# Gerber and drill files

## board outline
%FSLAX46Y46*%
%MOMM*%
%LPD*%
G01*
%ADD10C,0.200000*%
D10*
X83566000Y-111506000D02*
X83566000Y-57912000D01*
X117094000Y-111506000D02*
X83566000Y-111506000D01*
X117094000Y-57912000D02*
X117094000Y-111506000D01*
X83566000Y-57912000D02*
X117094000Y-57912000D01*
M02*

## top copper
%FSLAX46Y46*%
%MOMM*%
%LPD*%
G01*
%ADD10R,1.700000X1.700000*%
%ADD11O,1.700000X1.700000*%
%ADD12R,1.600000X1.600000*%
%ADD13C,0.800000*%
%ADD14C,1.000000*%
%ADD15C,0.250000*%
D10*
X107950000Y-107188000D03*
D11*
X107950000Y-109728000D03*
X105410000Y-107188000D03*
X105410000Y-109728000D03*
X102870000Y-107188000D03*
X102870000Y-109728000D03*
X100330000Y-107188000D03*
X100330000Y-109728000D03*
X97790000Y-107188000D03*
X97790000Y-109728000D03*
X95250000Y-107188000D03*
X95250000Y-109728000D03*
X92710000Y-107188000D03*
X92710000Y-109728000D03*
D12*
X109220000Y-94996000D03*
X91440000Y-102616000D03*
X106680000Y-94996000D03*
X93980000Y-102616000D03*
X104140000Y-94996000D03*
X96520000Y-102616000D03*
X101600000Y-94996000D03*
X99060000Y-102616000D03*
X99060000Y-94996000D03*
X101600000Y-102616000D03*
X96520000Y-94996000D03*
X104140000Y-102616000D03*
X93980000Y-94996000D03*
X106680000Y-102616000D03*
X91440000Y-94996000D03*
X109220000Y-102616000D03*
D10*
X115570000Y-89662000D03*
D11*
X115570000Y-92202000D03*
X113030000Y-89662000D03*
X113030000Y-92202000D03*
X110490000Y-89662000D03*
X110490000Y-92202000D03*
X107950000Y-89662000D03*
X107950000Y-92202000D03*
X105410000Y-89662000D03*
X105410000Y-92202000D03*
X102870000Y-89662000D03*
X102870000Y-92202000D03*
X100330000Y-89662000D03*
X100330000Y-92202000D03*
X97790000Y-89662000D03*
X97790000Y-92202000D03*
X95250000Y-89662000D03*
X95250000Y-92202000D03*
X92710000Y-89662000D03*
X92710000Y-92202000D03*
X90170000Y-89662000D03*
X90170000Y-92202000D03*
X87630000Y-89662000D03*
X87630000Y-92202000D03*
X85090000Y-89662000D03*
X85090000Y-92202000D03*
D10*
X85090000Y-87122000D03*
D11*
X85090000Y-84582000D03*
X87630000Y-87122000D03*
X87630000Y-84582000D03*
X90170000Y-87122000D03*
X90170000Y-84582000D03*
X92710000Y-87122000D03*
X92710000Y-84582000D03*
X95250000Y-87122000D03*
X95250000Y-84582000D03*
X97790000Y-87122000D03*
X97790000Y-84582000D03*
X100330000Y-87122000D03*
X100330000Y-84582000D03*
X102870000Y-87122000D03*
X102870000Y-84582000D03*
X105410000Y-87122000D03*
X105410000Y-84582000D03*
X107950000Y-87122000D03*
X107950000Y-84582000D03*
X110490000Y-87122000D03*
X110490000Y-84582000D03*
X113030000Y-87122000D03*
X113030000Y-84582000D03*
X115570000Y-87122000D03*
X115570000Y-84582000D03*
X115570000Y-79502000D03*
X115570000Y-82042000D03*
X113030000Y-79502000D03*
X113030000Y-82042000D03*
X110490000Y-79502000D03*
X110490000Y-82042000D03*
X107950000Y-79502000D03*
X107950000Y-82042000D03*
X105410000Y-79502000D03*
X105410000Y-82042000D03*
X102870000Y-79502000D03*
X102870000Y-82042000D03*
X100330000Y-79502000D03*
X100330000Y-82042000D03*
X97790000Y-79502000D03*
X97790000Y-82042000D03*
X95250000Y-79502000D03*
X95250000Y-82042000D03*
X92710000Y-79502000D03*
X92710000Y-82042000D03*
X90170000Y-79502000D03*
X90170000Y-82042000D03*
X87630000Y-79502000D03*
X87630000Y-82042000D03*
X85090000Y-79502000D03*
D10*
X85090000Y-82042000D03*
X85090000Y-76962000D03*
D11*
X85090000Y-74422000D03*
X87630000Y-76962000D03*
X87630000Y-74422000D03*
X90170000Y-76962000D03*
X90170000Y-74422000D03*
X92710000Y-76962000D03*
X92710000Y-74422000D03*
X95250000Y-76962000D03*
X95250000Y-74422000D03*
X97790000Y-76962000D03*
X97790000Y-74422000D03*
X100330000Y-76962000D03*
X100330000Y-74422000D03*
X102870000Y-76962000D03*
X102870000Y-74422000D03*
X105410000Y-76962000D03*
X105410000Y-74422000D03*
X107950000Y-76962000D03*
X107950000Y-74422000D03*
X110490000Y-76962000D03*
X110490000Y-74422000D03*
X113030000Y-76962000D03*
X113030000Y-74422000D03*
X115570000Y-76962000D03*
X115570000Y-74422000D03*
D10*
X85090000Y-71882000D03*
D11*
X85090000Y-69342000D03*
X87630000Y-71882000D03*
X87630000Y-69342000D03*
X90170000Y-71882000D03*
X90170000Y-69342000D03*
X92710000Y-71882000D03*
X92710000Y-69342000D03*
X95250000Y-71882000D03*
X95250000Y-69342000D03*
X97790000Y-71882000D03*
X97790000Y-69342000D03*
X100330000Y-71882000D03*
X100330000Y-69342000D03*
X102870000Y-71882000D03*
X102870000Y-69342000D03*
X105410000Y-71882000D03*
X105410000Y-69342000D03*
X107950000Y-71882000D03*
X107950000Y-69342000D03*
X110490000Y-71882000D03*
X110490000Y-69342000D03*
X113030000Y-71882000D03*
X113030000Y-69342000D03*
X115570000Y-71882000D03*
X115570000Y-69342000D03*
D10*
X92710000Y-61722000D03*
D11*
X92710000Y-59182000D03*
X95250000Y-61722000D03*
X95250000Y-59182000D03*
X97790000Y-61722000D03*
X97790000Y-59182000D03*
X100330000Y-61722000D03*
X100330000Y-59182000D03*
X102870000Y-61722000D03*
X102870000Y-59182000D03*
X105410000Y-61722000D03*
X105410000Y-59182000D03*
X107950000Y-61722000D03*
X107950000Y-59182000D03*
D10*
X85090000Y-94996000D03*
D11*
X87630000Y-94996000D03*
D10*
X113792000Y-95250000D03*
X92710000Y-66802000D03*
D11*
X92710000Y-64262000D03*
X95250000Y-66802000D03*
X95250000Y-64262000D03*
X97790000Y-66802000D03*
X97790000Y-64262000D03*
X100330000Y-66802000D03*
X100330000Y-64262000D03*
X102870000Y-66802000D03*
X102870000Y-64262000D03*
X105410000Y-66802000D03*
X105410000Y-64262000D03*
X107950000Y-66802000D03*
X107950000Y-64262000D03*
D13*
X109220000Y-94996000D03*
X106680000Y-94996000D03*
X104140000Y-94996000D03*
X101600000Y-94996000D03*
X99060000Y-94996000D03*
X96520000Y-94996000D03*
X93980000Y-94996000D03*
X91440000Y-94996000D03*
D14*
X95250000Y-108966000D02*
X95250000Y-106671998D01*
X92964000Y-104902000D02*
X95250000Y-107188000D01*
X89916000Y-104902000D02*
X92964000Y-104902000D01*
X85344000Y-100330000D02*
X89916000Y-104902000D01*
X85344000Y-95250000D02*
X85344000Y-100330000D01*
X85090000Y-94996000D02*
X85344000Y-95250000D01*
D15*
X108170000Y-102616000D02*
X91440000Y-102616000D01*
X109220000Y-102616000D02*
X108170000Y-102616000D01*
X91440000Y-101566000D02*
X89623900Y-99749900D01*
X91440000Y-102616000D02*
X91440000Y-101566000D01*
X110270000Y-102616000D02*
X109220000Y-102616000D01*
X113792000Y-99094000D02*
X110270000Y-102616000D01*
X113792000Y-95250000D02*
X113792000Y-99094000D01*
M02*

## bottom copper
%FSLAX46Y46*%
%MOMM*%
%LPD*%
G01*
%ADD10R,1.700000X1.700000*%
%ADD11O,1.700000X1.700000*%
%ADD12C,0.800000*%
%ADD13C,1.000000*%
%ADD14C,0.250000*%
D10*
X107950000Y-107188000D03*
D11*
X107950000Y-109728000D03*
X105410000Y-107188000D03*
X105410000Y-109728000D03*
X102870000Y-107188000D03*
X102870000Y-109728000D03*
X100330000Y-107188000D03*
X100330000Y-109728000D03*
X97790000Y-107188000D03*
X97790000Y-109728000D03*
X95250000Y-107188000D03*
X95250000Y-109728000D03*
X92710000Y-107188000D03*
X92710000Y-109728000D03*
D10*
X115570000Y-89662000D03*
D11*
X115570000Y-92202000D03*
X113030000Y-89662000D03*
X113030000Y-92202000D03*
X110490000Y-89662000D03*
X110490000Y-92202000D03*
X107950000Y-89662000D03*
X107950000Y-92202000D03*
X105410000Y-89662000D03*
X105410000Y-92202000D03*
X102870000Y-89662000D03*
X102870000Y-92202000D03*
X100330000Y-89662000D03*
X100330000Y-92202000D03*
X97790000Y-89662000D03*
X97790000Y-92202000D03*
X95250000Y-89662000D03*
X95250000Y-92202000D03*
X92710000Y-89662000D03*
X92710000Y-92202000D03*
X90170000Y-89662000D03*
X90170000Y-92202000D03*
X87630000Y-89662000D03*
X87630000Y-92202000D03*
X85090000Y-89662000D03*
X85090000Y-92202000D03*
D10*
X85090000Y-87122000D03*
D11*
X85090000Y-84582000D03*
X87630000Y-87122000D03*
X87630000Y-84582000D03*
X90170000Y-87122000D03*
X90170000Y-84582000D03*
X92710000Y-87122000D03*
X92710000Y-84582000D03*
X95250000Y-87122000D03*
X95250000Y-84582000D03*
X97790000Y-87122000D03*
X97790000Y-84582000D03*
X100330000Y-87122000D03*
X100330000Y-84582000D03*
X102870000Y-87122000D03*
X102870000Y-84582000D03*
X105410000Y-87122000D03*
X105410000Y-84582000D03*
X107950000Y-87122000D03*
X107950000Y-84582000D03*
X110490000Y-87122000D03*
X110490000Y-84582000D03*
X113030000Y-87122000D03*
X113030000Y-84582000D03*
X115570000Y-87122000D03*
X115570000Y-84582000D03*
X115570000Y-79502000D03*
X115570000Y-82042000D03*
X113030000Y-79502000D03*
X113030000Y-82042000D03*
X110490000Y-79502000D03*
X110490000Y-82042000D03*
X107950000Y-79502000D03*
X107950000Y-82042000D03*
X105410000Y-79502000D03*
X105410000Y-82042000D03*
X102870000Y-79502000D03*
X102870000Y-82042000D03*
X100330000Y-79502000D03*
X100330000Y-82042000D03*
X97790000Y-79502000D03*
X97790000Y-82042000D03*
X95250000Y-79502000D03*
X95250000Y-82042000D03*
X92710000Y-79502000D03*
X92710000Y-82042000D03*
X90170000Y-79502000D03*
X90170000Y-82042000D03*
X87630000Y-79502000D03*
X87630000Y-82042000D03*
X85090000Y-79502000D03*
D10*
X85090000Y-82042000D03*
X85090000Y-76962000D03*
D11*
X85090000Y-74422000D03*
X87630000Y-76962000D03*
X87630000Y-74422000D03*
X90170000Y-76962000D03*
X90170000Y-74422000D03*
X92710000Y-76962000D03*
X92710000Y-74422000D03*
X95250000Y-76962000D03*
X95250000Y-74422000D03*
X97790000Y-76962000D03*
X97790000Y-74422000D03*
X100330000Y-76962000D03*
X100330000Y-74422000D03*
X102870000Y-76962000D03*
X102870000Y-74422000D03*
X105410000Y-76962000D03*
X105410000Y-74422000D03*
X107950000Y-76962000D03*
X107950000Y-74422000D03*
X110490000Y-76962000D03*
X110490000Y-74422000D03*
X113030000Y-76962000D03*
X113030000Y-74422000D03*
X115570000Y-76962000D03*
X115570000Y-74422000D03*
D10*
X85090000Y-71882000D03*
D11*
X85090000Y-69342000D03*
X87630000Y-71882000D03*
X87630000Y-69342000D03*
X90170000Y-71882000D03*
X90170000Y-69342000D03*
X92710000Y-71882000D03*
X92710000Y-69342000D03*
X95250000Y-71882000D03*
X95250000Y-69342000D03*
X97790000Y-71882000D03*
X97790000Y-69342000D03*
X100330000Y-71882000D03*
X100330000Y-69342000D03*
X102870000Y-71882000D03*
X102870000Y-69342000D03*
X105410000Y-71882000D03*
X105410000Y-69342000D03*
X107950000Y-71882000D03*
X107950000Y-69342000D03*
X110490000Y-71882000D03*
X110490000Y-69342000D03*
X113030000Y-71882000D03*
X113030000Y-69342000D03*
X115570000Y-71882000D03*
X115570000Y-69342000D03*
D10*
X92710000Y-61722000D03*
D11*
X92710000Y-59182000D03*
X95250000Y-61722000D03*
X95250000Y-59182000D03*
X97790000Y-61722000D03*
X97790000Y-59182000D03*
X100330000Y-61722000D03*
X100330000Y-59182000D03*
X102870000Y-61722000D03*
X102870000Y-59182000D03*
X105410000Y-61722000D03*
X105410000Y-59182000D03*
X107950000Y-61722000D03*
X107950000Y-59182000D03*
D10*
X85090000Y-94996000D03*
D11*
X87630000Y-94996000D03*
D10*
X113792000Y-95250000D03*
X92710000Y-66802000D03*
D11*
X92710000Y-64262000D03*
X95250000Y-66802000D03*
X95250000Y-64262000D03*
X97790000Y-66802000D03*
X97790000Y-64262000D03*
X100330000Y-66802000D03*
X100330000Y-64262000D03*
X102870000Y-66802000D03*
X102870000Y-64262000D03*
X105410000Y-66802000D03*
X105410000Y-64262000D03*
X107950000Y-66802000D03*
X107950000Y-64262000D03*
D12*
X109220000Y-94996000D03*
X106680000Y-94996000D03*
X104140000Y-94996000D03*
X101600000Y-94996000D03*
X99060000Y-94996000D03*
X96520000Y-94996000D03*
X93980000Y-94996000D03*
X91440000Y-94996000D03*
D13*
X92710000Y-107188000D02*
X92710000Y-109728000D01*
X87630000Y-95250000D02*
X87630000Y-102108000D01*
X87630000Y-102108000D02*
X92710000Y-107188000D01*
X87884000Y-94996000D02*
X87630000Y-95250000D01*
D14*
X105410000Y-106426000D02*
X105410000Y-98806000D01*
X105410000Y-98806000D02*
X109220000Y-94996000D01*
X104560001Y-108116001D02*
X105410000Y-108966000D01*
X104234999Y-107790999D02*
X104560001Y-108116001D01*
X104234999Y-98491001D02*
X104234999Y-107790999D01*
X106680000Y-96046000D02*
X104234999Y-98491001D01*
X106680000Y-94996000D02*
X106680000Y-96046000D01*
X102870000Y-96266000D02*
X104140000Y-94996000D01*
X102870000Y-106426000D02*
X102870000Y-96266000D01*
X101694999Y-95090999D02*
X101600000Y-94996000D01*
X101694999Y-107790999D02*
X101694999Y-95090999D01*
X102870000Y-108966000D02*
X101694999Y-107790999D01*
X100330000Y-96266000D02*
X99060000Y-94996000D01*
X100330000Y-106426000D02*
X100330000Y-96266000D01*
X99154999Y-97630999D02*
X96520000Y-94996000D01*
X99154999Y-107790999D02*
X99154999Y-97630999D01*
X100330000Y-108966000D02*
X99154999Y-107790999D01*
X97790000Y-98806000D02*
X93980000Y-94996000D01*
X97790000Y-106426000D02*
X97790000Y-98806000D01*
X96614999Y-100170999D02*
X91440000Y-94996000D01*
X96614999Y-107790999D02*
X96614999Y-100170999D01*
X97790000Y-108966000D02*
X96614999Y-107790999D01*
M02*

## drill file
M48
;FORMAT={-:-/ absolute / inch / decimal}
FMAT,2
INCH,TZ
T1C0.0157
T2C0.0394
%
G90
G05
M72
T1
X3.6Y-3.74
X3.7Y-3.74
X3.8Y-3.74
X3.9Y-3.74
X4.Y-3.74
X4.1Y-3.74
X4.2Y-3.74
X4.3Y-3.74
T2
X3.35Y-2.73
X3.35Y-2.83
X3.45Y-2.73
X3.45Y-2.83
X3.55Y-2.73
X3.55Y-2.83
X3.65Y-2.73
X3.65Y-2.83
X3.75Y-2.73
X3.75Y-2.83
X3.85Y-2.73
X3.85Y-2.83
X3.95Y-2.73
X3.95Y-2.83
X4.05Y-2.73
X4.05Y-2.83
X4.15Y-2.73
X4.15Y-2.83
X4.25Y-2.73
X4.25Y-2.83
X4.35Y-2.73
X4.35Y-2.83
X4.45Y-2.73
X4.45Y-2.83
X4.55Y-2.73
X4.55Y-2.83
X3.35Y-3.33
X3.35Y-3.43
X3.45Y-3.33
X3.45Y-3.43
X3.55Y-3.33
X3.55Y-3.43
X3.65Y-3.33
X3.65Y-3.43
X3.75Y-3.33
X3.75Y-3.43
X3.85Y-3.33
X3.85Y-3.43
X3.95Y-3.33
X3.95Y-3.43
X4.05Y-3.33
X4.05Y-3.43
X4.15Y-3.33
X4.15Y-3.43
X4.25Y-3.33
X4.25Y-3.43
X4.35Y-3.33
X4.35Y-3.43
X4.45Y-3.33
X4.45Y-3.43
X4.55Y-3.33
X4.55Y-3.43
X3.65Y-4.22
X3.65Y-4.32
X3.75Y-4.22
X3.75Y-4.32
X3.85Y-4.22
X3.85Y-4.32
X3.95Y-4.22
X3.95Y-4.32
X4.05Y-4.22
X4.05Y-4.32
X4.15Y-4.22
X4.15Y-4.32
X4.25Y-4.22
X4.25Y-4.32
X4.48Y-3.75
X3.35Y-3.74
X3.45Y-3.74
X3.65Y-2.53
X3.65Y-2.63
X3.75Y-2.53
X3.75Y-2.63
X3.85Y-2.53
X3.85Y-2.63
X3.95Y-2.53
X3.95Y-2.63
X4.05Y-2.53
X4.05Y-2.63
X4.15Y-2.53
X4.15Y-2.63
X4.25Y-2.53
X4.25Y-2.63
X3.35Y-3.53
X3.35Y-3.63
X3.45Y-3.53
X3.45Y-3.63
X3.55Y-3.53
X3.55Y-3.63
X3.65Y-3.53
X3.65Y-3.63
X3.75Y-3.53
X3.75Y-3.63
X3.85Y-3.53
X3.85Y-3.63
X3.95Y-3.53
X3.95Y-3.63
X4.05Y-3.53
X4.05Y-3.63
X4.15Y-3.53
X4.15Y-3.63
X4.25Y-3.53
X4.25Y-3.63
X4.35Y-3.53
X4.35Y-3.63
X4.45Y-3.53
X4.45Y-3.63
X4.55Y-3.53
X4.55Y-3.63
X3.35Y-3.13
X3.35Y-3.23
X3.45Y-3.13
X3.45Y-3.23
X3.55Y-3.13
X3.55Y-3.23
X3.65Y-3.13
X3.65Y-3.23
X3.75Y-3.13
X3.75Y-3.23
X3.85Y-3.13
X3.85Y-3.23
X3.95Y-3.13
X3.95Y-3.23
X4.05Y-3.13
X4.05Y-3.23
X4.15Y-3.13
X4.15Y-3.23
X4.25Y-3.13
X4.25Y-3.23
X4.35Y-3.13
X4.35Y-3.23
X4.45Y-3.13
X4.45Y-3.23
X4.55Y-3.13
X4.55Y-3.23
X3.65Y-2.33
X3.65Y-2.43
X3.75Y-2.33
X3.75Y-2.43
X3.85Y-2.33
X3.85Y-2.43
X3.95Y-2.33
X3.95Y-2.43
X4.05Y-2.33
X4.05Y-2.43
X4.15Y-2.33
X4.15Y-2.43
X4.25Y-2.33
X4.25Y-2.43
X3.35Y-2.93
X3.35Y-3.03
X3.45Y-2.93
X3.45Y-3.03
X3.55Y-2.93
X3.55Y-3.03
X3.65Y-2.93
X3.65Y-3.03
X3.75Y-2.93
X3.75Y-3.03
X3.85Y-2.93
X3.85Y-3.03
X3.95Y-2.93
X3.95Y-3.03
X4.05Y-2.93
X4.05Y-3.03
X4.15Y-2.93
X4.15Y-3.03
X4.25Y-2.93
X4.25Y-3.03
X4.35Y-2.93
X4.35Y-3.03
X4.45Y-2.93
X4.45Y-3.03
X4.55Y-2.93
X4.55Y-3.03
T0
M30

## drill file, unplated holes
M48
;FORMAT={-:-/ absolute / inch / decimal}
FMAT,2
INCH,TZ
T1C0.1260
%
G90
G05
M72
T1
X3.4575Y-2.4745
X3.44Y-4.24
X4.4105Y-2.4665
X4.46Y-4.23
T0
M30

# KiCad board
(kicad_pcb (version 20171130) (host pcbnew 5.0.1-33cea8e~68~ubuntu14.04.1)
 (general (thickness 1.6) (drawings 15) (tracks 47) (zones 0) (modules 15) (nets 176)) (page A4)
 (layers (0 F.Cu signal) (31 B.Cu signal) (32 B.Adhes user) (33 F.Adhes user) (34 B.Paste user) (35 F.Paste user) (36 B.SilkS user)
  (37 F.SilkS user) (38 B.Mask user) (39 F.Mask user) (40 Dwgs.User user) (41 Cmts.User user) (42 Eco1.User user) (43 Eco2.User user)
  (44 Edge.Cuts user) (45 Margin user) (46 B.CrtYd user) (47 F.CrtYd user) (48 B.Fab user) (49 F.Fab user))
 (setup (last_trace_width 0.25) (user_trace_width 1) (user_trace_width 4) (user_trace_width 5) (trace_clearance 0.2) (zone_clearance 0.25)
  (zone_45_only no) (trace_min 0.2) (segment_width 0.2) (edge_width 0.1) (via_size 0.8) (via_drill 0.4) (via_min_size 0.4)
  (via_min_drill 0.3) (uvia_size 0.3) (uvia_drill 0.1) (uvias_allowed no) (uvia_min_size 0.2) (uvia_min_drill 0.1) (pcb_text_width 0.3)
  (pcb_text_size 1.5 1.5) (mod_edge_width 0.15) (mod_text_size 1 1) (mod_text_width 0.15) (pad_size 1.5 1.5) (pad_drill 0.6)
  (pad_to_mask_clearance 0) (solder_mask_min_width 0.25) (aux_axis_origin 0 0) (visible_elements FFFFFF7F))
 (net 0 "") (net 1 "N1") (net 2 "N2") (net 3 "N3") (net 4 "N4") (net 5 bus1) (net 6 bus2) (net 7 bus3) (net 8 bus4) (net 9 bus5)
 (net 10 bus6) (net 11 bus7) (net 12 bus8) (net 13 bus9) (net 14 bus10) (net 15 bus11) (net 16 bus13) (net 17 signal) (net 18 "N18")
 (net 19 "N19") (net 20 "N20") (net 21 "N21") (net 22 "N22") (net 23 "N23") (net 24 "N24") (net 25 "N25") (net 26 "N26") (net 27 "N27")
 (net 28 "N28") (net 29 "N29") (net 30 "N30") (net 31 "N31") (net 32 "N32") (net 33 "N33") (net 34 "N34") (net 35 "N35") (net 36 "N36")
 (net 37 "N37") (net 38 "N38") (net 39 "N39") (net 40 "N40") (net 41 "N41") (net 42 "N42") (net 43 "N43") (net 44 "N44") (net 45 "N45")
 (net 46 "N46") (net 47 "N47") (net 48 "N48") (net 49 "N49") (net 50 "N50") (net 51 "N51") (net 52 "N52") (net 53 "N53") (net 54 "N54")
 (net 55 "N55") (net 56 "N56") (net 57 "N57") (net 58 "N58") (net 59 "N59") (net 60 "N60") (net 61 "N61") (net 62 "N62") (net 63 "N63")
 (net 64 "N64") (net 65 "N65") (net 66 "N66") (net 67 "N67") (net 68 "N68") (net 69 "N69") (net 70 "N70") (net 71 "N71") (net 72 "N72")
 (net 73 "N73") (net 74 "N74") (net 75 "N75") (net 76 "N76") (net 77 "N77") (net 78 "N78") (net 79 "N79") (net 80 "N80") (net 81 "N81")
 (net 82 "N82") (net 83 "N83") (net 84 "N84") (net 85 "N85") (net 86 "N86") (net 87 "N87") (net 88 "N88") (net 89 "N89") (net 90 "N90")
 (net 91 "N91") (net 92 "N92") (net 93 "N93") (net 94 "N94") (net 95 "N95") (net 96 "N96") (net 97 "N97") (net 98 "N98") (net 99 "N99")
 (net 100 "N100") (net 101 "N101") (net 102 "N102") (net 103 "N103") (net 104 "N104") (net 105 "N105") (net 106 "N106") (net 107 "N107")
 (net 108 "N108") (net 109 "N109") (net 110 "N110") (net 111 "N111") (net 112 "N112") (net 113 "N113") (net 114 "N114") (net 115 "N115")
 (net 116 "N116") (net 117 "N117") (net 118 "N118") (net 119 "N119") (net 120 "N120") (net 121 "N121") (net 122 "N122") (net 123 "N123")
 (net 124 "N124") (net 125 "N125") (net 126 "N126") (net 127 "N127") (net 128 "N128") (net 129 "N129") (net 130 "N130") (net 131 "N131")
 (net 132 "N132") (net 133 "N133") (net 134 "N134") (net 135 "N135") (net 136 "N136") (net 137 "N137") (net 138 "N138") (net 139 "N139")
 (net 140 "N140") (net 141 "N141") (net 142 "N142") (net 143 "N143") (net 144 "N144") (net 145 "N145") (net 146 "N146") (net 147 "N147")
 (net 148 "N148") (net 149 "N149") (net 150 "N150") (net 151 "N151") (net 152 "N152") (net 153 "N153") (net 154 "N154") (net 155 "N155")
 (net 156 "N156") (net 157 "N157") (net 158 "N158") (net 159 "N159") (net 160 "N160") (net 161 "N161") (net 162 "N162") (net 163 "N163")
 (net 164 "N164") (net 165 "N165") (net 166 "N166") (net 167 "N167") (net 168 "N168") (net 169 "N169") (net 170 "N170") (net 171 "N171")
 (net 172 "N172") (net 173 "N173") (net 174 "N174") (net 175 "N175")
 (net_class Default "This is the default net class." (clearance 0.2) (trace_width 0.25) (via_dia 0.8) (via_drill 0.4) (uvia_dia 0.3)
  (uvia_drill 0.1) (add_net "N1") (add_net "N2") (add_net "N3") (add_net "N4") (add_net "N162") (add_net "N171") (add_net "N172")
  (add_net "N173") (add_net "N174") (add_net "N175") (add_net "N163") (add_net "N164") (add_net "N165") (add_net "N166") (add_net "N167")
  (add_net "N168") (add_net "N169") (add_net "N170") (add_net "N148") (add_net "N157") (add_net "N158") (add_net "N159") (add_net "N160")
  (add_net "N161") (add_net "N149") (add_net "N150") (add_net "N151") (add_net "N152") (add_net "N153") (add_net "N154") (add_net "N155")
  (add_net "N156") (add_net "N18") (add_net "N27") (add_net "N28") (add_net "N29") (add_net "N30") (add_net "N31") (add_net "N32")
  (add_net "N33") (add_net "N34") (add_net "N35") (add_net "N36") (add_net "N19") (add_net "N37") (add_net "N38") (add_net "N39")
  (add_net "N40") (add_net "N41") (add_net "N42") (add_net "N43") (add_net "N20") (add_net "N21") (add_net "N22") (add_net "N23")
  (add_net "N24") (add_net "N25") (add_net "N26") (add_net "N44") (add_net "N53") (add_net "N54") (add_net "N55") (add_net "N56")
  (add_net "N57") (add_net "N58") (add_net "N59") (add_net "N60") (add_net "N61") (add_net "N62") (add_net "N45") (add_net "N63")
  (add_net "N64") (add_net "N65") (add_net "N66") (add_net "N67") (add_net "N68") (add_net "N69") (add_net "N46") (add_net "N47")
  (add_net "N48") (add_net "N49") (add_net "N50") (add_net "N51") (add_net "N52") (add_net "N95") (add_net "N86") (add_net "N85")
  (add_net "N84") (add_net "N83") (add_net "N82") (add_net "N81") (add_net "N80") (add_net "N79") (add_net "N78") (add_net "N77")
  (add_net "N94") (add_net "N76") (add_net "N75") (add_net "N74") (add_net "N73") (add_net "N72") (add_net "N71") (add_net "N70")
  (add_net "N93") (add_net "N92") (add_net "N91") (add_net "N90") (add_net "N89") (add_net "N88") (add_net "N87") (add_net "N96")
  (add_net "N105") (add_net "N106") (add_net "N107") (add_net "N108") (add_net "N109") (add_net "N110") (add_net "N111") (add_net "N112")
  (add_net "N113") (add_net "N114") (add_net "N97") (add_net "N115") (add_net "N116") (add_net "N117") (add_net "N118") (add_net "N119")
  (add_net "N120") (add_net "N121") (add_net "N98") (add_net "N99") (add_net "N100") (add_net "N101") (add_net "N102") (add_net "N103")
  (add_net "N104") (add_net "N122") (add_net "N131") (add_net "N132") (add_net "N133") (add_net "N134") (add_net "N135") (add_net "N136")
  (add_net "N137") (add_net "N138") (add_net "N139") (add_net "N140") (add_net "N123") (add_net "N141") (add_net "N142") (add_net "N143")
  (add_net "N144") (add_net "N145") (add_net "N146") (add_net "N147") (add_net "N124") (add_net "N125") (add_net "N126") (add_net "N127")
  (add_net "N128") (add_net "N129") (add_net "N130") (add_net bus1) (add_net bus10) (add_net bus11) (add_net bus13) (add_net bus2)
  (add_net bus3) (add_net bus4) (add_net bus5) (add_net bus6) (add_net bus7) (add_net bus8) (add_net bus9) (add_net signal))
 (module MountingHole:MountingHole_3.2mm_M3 (layer F.Cu) (at 87.376 107.696)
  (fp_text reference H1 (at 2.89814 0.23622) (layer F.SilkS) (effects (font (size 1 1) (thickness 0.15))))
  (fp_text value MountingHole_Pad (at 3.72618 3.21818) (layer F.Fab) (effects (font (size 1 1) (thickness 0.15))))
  (pad 1 np_thru_hole circle (at 0 0) (size 3.2 3.2) (drill 3.2) (layers *.Cu *.Mask) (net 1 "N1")))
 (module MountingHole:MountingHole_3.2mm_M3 (layer F.Cu) (at 113.284 107.442)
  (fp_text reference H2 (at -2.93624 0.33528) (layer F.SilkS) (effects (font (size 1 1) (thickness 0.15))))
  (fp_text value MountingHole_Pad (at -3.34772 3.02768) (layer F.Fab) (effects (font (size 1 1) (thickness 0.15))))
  (pad 1 np_thru_hole circle (at 0 0) (size 3.2 3.2) (drill 3.2) (layers *.Cu *.Mask) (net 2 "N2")))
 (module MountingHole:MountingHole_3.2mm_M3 (layer F.Cu) (at 112.0267 62.6491)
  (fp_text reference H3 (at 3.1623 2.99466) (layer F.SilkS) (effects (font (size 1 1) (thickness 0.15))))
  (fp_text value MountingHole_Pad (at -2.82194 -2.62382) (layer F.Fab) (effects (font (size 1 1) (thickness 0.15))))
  (pad 1 np_thru_hole circle (at 0 0) (size 3.2 3.2) (drill 3.2) (layers *.Cu *.Mask) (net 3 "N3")))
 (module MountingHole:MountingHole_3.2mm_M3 (layer F.Cu) (at 87.8205 62.8523)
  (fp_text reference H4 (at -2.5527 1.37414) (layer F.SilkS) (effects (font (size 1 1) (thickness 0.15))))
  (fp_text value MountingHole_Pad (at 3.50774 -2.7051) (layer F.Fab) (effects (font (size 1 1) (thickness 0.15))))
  (pad 1 np_thru_hole circle (at 0 0) (size 3.2 3.2) (drill 3.2) (layers *.Cu *.Mask) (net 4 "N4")))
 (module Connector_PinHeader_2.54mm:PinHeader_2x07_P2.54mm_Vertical (layer F.Cu) (at 107.95 107.188 270)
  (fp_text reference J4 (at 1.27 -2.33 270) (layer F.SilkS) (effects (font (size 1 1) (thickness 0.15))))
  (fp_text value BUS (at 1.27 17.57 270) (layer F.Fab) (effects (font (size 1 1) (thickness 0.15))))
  (pad 1 thru_hole rect (at 0 0 270) (size 1.7 1.7) (drill 1) (layers *.Cu *.Mask) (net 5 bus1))
  (pad 2 thru_hole oval (at 2.54 0 270) (size 1.7 1.7) (drill 1) (layers *.Cu *.Mask) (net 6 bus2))
  (pad 3 thru_hole oval (at 0 2.54 270) (size 1.7 1.7) (drill 1) (layers *.Cu *.Mask) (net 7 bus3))
  (pad 4 thru_hole oval (at 2.54 2.54 270) (size 1.7 1.7) (drill 1) (layers *.Cu *.Mask) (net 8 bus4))
  (pad 5 thru_hole oval (at 0 5.08 270) (size 1.7 1.7) (drill 1) (layers *.Cu *.Mask) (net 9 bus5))
  (pad 6 thru_hole oval (at 2.54 5.08 270) (size 1.7 1.7) (drill 1) (layers *.Cu *.Mask) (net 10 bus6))
  (pad 7 thru_hole oval (at 0 7.62 270) (size 1.7 1.7) (drill 1) (layers *.Cu *.Mask) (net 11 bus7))
  (pad 8 thru_hole oval (at 2.54 7.62 270) (size 1.7 1.7) (drill 1) (layers *.Cu *.Mask) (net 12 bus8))
  (pad 9 thru_hole oval (at 0 10.16 270) (size 1.7 1.7) (drill 1) (layers *.Cu *.Mask) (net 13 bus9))
  (pad 10 thru_hole oval (at 2.54 10.16 270) (size 1.7 1.7) (drill 1) (layers *.Cu *.Mask) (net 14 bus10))
  (pad 11 thru_hole oval (at 0 12.7 270) (size 1.7 1.7) (drill 1) (layers *.Cu *.Mask) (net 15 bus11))
  (pad 12 thru_hole oval (at 2.54 12.7 270) (size 1.7 1.7) (drill 1) (layers *.Cu *.Mask) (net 15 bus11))
  (pad 13 thru_hole oval (at 0 15.24 270) (size 1.7 1.7) (drill 1) (layers *.Cu *.Mask) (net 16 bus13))
  (pad 14 thru_hole oval (at 2.54 15.24 270) (size 1.7 1.7) (drill 1) (layers *.Cu *.Mask) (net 16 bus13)))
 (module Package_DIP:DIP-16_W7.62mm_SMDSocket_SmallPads (layer F.Cu) (at 100.33 98.806 270)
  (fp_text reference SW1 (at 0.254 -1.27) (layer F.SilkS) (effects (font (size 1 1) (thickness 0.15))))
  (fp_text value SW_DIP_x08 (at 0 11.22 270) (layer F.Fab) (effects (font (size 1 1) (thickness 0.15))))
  (pad 1 smd rect (at -3.81 -8.89 270) (size 1.6 1.6) (layers F.Cu F.Paste F.Mask) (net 7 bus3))
  (pad 9 smd rect (at 3.81 8.89 270) (size 1.6 1.6) (layers F.Cu F.Paste F.Mask) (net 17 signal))
  (pad 2 smd rect (at -3.81 -6.35 270) (size 1.6 1.6) (layers F.Cu F.Paste F.Mask) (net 8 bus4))
  (pad 10 smd rect (at 3.81 6.35 270) (size 1.6 1.6) (layers F.Cu F.Paste F.Mask) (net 17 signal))
  (pad 3 smd rect (at -3.81 -3.81 270) (size 1.6 1.6) (layers F.Cu F.Paste F.Mask) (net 9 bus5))
  (pad 11 smd rect (at 3.81 3.81 270) (size 1.6 1.6) (layers F.Cu F.Paste F.Mask) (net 17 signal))
  (pad 4 smd rect (at -3.81 -1.27 270) (size 1.6 1.6) (layers F.Cu F.Paste F.Mask) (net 10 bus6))
  (pad 12 smd rect (at 3.81 1.27 270) (size 1.6 1.6) (layers F.Cu F.Paste F.Mask) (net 17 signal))
  (pad 5 smd rect (at -3.81 1.27 270) (size 1.6 1.6) (layers F.Cu F.Paste F.Mask) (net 11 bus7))
  (pad 13 smd rect (at 3.81 -1.27 270) (size 1.6 1.6) (layers F.Cu F.Paste F.Mask) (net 17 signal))
  (pad 6 smd rect (at -3.81 3.81 270) (size 1.6 1.6) (layers F.Cu F.Paste F.Mask) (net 12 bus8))
  (pad 14 smd rect (at 3.81 -3.81 270) (size 1.6 1.6) (layers F.Cu F.Paste F.Mask) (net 17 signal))
  (pad 7 smd rect (at -3.81 6.35 270) (size 1.6 1.6) (layers F.Cu F.Paste F.Mask) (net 13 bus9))
  (pad 15 smd rect (at 3.81 -6.35 270) (size 1.6 1.6) (layers F.Cu F.Paste F.Mask) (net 17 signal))
  (pad 8 smd rect (at -3.81 8.89 270) (size 1.6 1.6) (layers F.Cu F.Paste F.Mask) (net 14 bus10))
  (pad 16 smd rect (at 3.81 -8.89 270) (size 1.6 1.6) (layers F.Cu F.Paste F.Mask) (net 17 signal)))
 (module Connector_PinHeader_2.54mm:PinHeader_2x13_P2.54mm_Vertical (layer F.Cu) (at 115.57 89.662 270)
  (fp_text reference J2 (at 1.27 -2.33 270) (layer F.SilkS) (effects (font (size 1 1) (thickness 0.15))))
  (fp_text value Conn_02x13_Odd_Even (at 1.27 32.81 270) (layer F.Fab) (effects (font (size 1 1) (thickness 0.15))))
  (pad 1 thru_hole rect (at 0 0 270) (size 1.7 1.7) (drill 1) (layers *.Cu *.Mask) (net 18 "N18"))
  (pad 2 thru_hole oval (at 2.54 0 270) (size 1.7 1.7) (drill 1) (layers *.Cu *.Mask) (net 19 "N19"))
  (pad 3 thru_hole oval (at 0 2.54 270) (size 1.7 1.7) (drill 1) (layers *.Cu *.Mask) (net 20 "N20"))
  (pad 4 thru_hole oval (at 2.54 2.54 270) (size 1.7 1.7) (drill 1) (layers *.Cu *.Mask) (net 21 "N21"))
  (pad 5 thru_hole oval (at 0 5.08 270) (size 1.7 1.7) (drill 1) (layers *.Cu *.Mask) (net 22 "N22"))
  (pad 6 thru_hole oval (at 2.54 5.08 270) (size 1.7 1.7) (drill 1) (layers *.Cu *.Mask) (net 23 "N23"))
  (pad 7 thru_hole oval (at 0 7.62 270) (size 1.7 1.7) (drill 1) (layers *.Cu *.Mask) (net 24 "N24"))
  (pad 8 thru_hole oval (at 2.54 7.62 270) (size 1.7 1.7) (drill 1) (layers *.Cu *.Mask) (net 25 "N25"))
  (pad 9 thru_hole oval (at 0 10.16 270) (size 1.7 1.7) (drill 1) (layers *.Cu *.Mask) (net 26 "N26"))
  (pad 10 thru_hole oval (at 2.54 10.16 270) (size 1.7 1.7) (drill 1) (layers *.Cu *.Mask) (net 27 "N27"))
  (pad 11 thru_hole oval (at 0 12.7 270) (size 1.7 1.7) (drill 1) (layers *.Cu *.Mask) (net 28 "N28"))
  (pad 12 thru_hole oval (at 2.54 12.7 270) (size 1.7 1.7) (drill 1) (layers *.Cu *.Mask) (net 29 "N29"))
  (pad 13 thru_hole oval (at 0 15.24 270) (size 1.7 1.7) (drill 1) (layers *.Cu *.Mask) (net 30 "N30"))
  (pad 14 thru_hole oval (at 2.54 15.24 270) (size 1.7 1.7) (drill 1) (layers *.Cu *.Mask) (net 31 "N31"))
  (pad 15 thru_hole oval (at 0 17.78 270) (size 1.7 1.7) (drill 1) (layers *.Cu *.Mask) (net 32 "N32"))
  (pad 16 thru_hole oval (at 2.54 17.78 270) (size 1.7 1.7) (drill 1) (layers *.Cu *.Mask) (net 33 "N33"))
  (pad 17 thru_hole oval (at 0 20.32 270) (size 1.7 1.7) (drill 1) (layers *.Cu *.Mask) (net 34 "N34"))
  (pad 18 thru_hole oval (at 2.54 20.32 270) (size 1.7 1.7) (drill 1) (layers *.Cu *.Mask) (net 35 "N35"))
  (pad 19 thru_hole oval (at 0 22.86 270) (size 1.7 1.7) (drill 1) (layers *.Cu *.Mask) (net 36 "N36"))
  (pad 20 thru_hole oval (at 2.54 22.86 270) (size 1.7 1.7) (drill 1) (layers *.Cu *.Mask) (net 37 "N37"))
  (pad 21 thru_hole oval (at 0 25.4 270) (size 1.7 1.7) (drill 1) (layers *.Cu *.Mask) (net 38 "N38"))
  (pad 22 thru_hole oval (at 2.54 25.4 270) (size 1.7 1.7) (drill 1) (layers *.Cu *.Mask) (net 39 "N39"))
  (pad 23 thru_hole oval (at 0 27.94 270) (size 1.7 1.7) (drill 1) (layers *.Cu *.Mask) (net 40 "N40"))
  (pad 24 thru_hole oval (at 2.54 27.94 270) (size 1.7 1.7) (drill 1) (layers *.Cu *.Mask) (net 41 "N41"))
  (pad 25 thru_hole oval (at 0 30.48 270) (size 1.7 1.7) (drill 1) (layers *.Cu *.Mask) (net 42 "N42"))
  (pad 26 thru_hole oval (at 2.54 30.48 270) (size 1.7 1.7) (drill 1) (layers *.Cu *.Mask) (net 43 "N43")))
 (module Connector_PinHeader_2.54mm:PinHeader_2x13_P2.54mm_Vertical (layer F.Cu) (at 85.09 87.122 90)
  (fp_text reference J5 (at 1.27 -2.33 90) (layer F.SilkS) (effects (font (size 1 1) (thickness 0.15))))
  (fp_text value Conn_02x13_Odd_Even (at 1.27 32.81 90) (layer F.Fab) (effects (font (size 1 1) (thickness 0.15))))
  (pad 1 thru_hole rect (at 0 0 90) (size 1.7 1.7) (drill 1) (layers *.Cu *.Mask) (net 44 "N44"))
  (pad 2 thru_hole oval (at 2.54 0 90) (size 1.7 1.7) (drill 1) (layers *.Cu *.Mask) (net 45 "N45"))
  (pad 3 thru_hole oval (at 0 2.54 90) (size 1.7 1.7) (drill 1) (layers *.Cu *.Mask) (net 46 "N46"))
  (pad 4 thru_hole oval (at 2.54 2.54 90) (size 1.7 1.7) (drill 1) (layers *.Cu *.Mask) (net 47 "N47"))
  (pad 5 thru_hole oval (at 0 5.08 90) (size 1.7 1.7) (drill 1) (layers *.Cu *.Mask) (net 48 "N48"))
  (pad 6 thru_hole oval (at 2.54 5.08 90) (size 1.7 1.7) (drill 1) (layers *.Cu *.Mask) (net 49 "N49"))
  (pad 7 thru_hole oval (at 0 7.62 90) (size 1.7 1.7) (drill 1) (layers *.Cu *.Mask) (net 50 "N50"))
  (pad 8 thru_hole oval (at 2.54 7.62 90) (size 1.7 1.7) (drill 1) (layers *.Cu *.Mask) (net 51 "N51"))
  (pad 9 thru_hole oval (at 0 10.16 90) (size 1.7 1.7) (drill 1) (layers *.Cu *.Mask) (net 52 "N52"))
  (pad 10 thru_hole oval (at 2.54 10.16 90) (size 1.7 1.7) (drill 1) (layers *.Cu *.Mask) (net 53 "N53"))
  (pad 11 thru_hole oval (at 0 12.7 90) (size 1.7 1.7) (drill 1) (layers *.Cu *.Mask) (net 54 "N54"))
  (pad 12 thru_hole oval (at 2.54 12.7 90) (size 1.7 1.7) (drill 1) (layers *.Cu *.Mask) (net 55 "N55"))
  (pad 13 thru_hole oval (at 0 15.24 90) (size 1.7 1.7) (drill 1) (layers *.Cu *.Mask) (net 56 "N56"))
  (pad 14 thru_hole oval (at 2.54 15.24 90) (size 1.7 1.7) (drill 1) (layers *.Cu *.Mask) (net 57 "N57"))
  (pad 15 thru_hole oval (at 0 17.78 90) (size 1.7 1.7) (drill 1) (layers *.Cu *.Mask) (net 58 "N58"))
  (pad 16 thru_hole oval (at 2.54 17.78 90) (size 1.7 1.7) (drill 1) (layers *.Cu *.Mask) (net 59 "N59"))
  (pad 17 thru_hole oval (at 0 20.32 90) (size 1.7 1.7) (drill 1) (layers *.Cu *.Mask) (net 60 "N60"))
  (pad 18 thru_hole oval (at 2.54 20.32 90) (size 1.7 1.7) (drill 1) (layers *.Cu *.Mask) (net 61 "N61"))
  (pad 19 thru_hole oval (at 0 22.86 90) (size 1.7 1.7) (drill 1) (layers *.Cu *.Mask) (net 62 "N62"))
  (pad 20 thru_hole oval (at 2.54 22.86 90) (size 1.7 1.7) (drill 1) (layers *.Cu *.Mask) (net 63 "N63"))
  (pad 21 thru_hole oval (at 0 25.4 90) (size 1.7 1.7) (drill 1) (layers *.Cu *.Mask) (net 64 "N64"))
  (pad 22 thru_hole oval (at 2.54 25.4 90) (size 1.7 1.7) (drill 1) (layers *.Cu *.Mask) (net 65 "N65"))
  (pad 23 thru_hole oval (at 0 27.94 90) (size 1.7 1.7) (drill 1) (layers *.Cu *.Mask) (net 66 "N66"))
  (pad 24 thru_hole oval (at 2.54 27.94 90) (size 1.7 1.7) (drill 1) (layers *.Cu *.Mask) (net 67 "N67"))
  (pad 25 thru_hole oval (at 0 30.48 90) (size 1.7 1.7) (drill 1) (layers *.Cu *.Mask) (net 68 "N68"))
  (pad 26 thru_hole oval (at 2.54 30.48 90) (size 1.7 1.7) (drill 1) (layers *.Cu *.Mask) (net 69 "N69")))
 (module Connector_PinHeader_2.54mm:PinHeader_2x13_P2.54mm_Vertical (layer F.Cu) (at 85.09 82.042 90)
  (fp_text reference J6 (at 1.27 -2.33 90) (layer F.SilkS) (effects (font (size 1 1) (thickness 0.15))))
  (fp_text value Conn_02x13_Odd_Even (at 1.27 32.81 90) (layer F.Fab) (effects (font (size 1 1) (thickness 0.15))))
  (pad 26 thru_hole oval (at 2.54 30.48 90) (size 1.7 1.7) (drill 1) (layers *.Cu *.Mask) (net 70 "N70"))
  (pad 25 thru_hole oval (at 0 30.48 90) (size 1.7 1.7) (drill 1) (layers *.Cu *.Mask) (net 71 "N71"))
  (pad 24 thru_hole oval (at 2.54 27.94 90) (size 1.7 1.7) (drill 1) (layers *.Cu *.Mask) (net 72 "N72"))
  (pad 23 thru_hole oval (at 0 27.94 90) (size 1.7 1.7) (drill 1) (layers *.Cu *.Mask) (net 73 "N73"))
  (pad 22 thru_hole oval (at 2.54 25.4 90) (size 1.7 1.7) (drill 1) (layers *.Cu *.Mask) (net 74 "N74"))
  (pad 21 thru_hole oval (at 0 25.4 90) (size 1.7 1.7) (drill 1) (layers *.Cu *.Mask) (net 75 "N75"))
  (pad 20 thru_hole oval (at 2.54 22.86 90) (size 1.7 1.7) (drill 1) (layers *.Cu *.Mask) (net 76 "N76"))
  (pad 19 thru_hole oval (at 0 22.86 90) (size 1.7 1.7) (drill 1) (layers *.Cu *.Mask) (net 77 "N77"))
  (pad 18 thru_hole oval (at 2.54 20.32 90) (size 1.7 1.7) (drill 1) (layers *.Cu *.Mask) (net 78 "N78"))
  (pad 17 thru_hole oval (at 0 20.32 90) (size 1.7 1.7) (drill 1) (layers *.Cu *.Mask) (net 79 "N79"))
  (pad 16 thru_hole oval (at 2.54 17.78 90) (size 1.7 1.7) (drill 1) (layers *.Cu *.Mask) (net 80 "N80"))
  (pad 15 thru_hole oval (at 0 17.78 90) (size 1.7 1.7) (drill 1) (layers *.Cu *.Mask) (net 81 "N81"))
  (pad 14 thru_hole oval (at 2.54 15.24 90) (size 1.7 1.7) (drill 1) (layers *.Cu *.Mask) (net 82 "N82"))
  (pad 13 thru_hole oval (at 0 15.24 90) (size 1.7 1.7) (drill 1) (layers *.Cu *.Mask) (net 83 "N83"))
  (pad 12 thru_hole oval (at 2.54 12.7 90) (size 1.7 1.7) (drill 1) (layers *.Cu *.Mask) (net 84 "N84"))
  (pad 11 thru_hole oval (at 0 12.7 90) (size 1.7 1.7) (drill 1) (layers *.Cu *.Mask) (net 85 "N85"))
  (pad 10 thru_hole oval (at 2.54 10.16 90) (size 1.7 1.7) (drill 1) (layers *.Cu *.Mask) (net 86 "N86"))
  (pad 9 thru_hole oval (at 0 10.16 90) (size 1.7 1.7) (drill 1) (layers *.Cu *.Mask) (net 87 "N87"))
  (pad 8 thru_hole oval (at 2.54 7.62 90) (size 1.7 1.7) (drill 1) (layers *.Cu *.Mask) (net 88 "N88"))
  (pad 7 thru_hole oval (at 0 7.62 90) (size 1.7 1.7) (drill 1) (layers *.Cu *.Mask) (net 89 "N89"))
  (pad 6 thru_hole oval (at 2.54 5.08 90) (size 1.7 1.7) (drill 1) (layers *.Cu *.Mask) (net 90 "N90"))
  (pad 5 thru_hole oval (at 0 5.08 90) (size 1.7 1.7) (drill 1) (layers *.Cu *.Mask) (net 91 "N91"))
  (pad 4 thru_hole oval (at 2.54 2.54 90) (size 1.7 1.7) (drill 1) (layers *.Cu *.Mask) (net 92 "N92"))
  (pad 3 thru_hole oval (at 0 2.54 90) (size 1.7 1.7) (drill 1) (layers *.Cu *.Mask) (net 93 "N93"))
  (pad 2 thru_hole oval (at 2.54 0 90) (size 1.7 1.7) (drill 1) (layers *.Cu *.Mask) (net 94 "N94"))
  (pad 1 thru_hole rect (at 0 0 90) (size 1.7 1.7) (drill 1) (layers *.Cu *.Mask) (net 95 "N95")))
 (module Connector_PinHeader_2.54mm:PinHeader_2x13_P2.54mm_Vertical (layer F.Cu) (at 85.09 76.962 90)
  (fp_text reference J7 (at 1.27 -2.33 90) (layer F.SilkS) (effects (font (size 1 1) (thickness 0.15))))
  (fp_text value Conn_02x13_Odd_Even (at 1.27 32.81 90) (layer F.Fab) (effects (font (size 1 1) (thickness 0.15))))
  (pad 1 thru_hole rect (at 0 0 90) (size 1.7 1.7) (drill 1) (layers *.Cu *.Mask) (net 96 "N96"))
  (pad 2 thru_hole oval (at 2.54 0 90) (size 1.7 1.7) (drill 1) (layers *.Cu *.Mask) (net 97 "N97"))
  (pad 3 thru_hole oval (at 0 2.54 90) (size 1.7 1.7) (drill 1) (layers *.Cu *.Mask) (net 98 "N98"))
  (pad 4 thru_hole oval (at 2.54 2.54 90) (size 1.7 1.7) (drill 1) (layers *.Cu *.Mask) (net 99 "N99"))
  (pad 5 thru_hole oval (at 0 5.08 90) (size 1.7 1.7) (drill 1) (layers *.Cu *.Mask) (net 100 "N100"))
  (pad 6 thru_hole oval (at 2.54 5.08 90) (size 1.7 1.7) (drill 1) (layers *.Cu *.Mask) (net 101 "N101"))
  (pad 7 thru_hole oval (at 0 7.62 90) (size 1.7 1.7) (drill 1) (layers *.Cu *.Mask) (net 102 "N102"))
  (pad 8 thru_hole oval (at 2.54 7.62 90) (size 1.7 1.7) (drill 1) (layers *.Cu *.Mask) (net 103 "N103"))
  (pad 9 thru_hole oval (at 0 10.16 90) (size 1.7 1.7) (drill 1) (layers *.Cu *.Mask) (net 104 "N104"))
  (pad 10 thru_hole oval (at 2.54 10.16 90) (size 1.7 1.7) (drill 1) (layers *.Cu *.Mask) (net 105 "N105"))
  (pad 11 thru_hole oval (at 0 12.7 90) (size 1.7 1.7) (drill 1) (layers *.Cu *.Mask) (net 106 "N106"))
  (pad 12 thru_hole oval (at 2.54 12.7 90) (size 1.7 1.7) (drill 1) (layers *.Cu *.Mask) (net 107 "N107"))
  (pad 13 thru_hole oval (at 0 15.24 90) (size 1.7 1.7) (drill 1) (layers *.Cu *.Mask) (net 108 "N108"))
  (pad 14 thru_hole oval (at 2.54 15.24 90) (size 1.7 1.7) (drill 1) (layers *.Cu *.Mask) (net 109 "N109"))
  (pad 15 thru_hole oval (at 0 17.78 90) (size 1.7 1.7) (drill 1) (layers *.Cu *.Mask) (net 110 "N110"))
  (pad 16 thru_hole oval (at 2.54 17.78 90) (size 1.7 1.7) (drill 1) (layers *.Cu *.Mask) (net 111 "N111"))
  (pad 17 thru_hole oval (at 0 20.32 90) (size 1.7 1.7) (drill 1) (layers *.Cu *.Mask) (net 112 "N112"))
  (pad 18 thru_hole oval (at 2.54 20.32 90) (size 1.7 1.7) (drill 1) (layers *.Cu *.Mask) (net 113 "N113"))
  (pad 19 thru_hole oval (at 0 22.86 90) (size 1.7 1.7) (drill 1) (layers *.Cu *.Mask) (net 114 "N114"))
  (pad 20 thru_hole oval (at 2.54 22.86 90) (size 1.7 1.7) (drill 1) (layers *.Cu *.Mask) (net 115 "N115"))
  (pad 21 thru_hole oval (at 0 25.4 90) (size 1.7 1.7) (drill 1) (layers *.Cu *.Mask) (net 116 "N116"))
  (pad 22 thru_hole oval (at 2.54 25.4 90) (size 1.7 1.7) (drill 1) (layers *.Cu *.Mask) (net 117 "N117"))
  (pad 23 thru_hole oval (at 0 27.94 90) (size 1.7 1.7) (drill 1) (layers *.Cu *.Mask) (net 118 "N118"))
  (pad 24 thru_hole oval (at 2.54 27.94 90) (size 1.7 1.7) (drill 1) (layers *.Cu *.Mask) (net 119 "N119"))
  (pad 25 thru_hole oval (at 0 30.48 90) (size 1.7 1.7) (drill 1) (layers *.Cu *.Mask) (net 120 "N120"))
  (pad 26 thru_hole oval (at 2.54 30.48 90) (size 1.7 1.7) (drill 1) (layers *.Cu *.Mask) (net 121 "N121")))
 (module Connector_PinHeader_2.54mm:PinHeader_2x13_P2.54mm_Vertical (layer F.Cu) (at 85.09 71.882 90)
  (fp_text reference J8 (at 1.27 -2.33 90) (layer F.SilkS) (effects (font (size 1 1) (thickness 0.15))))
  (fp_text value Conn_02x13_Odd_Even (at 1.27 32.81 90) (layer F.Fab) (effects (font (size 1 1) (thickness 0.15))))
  (pad 1 thru_hole rect (at 0 0 90) (size 1.7 1.7) (drill 1) (layers *.Cu *.Mask) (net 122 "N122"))
  (pad 2 thru_hole oval (at 2.54 0 90) (size 1.7 1.7) (drill 1) (layers *.Cu *.Mask) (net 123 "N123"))
  (pad 3 thru_hole oval (at 0 2.54 90) (size 1.7 1.7) (drill 1) (layers *.Cu *.Mask) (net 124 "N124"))
  (pad 4 thru_hole oval (at 2.54 2.54 90) (size 1.7 1.7) (drill 1) (layers *.Cu *.Mask) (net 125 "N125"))
  (pad 5 thru_hole oval (at 0 5.08 90) (size 1.7 1.7) (drill 1) (layers *.Cu *.Mask) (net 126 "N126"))
  (pad 6 thru_hole oval (at 2.54 5.08 90) (size 1.7 1.7) (drill 1) (layers *.Cu *.Mask) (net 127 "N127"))
  (pad 7 thru_hole oval (at 0 7.62 90) (size 1.7 1.7) (drill 1) (layers *.Cu *.Mask) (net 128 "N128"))
  (pad 8 thru_hole oval (at 2.54 7.62 90) (size 1.7 1.7) (drill 1) (layers *.Cu *.Mask) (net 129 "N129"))
  (pad 9 thru_hole oval (at 0 10.16 90) (size 1.7 1.7) (drill 1) (layers *.Cu *.Mask) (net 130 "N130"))
  (pad 10 thru_hole oval (at 2.54 10.16 90) (size 1.7 1.7) (drill 1) (layers *.Cu *.Mask) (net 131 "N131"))
  (pad 11 thru_hole oval (at 0 12.7 90) (size 1.7 1.7) (drill 1) (layers *.Cu *.Mask) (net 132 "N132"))
  (pad 12 thru_hole oval (at 2.54 12.7 90) (size 1.7 1.7) (drill 1) (layers *.Cu *.Mask) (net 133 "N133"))
  (pad 13 thru_hole oval (at 0 15.24 90) (size 1.7 1.7) (drill 1) (layers *.Cu *.Mask) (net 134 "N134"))
  (pad 14 thru_hole oval (at 2.54 15.24 90) (size 1.7 1.7) (drill 1) (layers *.Cu *.Mask) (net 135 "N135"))
  (pad 15 thru_hole oval (at 0 17.78 90) (size 1.7 1.7) (drill 1) (layers *.Cu *.Mask) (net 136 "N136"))
  (pad 16 thru_hole oval (at 2.54 17.78 90) (size 1.7 1.7) (drill 1) (layers *.Cu *.Mask) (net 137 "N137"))
  (pad 17 thru_hole oval (at 0 20.32 90) (size 1.7 1.7) (drill 1) (layers *.Cu *.Mask) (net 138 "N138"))
  (pad 18 thru_hole oval (at 2.54 20.32 90) (size 1.7 1.7) (drill 1) (layers *.Cu *.Mask) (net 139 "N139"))
  (pad 19 thru_hole oval (at 0 22.86 90) (size 1.7 1.7) (drill 1) (layers *.Cu *.Mask) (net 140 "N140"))
  (pad 20 thru_hole oval (at 2.54 22.86 90) (size 1.7 1.7) (drill 1) (layers *.Cu *.Mask) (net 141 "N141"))
  (pad 21 thru_hole oval (at 0 25.4 90) (size 1.7 1.7) (drill 1) (layers *.Cu *.Mask) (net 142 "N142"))
  (pad 22 thru_hole oval (at 2.54 25.4 90) (size 1.7 1.7) (drill 1) (layers *.Cu *.Mask) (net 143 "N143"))
  (pad 23 thru_hole oval (at 0 27.94 90) (size 1.7 1.7) (drill 1) (layers *.Cu *.Mask) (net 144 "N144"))
  (pad 24 thru_hole oval (at 2.54 27.94 90) (size 1.7 1.7) (drill 1) (layers *.Cu *.Mask) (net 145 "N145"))
  (pad 25 thru_hole oval (at 0 30.48 90) (size 1.7 1.7) (drill 1) (layers *.Cu *.Mask) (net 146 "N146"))
  (pad 26 thru_hole oval (at 2.54 30.48 90) (size 1.7 1.7) (drill 1) (layers *.Cu *.Mask) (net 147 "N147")))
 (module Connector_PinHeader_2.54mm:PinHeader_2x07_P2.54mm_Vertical (layer F.Cu) (at 92.71 61.722 90)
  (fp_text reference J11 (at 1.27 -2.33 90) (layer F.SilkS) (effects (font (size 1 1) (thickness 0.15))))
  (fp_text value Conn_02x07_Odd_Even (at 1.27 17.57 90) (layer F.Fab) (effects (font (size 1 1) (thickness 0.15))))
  (pad 1 thru_hole rect (at 0 0 90) (size 1.7 1.7) (drill 1) (layers *.Cu *.Mask) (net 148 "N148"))
  (pad 2 thru_hole oval (at 2.54 0 90) (size 1.7 1.7) (drill 1) (layers *.Cu *.Mask) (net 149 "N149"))
  (pad 3 thru_hole oval (at 0 2.54 90) (size 1.7 1.7) (drill 1) (layers *.Cu *.Mask) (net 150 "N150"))
  (pad 4 thru_hole oval (at 2.54 2.54 90) (size 1.7 1.7) (drill 1) (layers *.Cu *.Mask) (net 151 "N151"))
  (pad 5 thru_hole oval (at 0 5.08 90) (size 1.7 1.7) (drill 1) (layers *.Cu *.Mask) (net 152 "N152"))
  (pad 6 thru_hole oval (at 2.54 5.08 90) (size 1.7 1.7) (drill 1) (layers *.Cu *.Mask) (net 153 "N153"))
  (pad 7 thru_hole oval (at 0 7.62 90) (size 1.7 1.7) (drill 1) (layers *.Cu *.Mask) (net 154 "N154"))
  (pad 8 thru_hole oval (at 2.54 7.62 90) (size 1.7 1.7) (drill 1) (layers *.Cu *.Mask) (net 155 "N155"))
  (pad 9 thru_hole oval (at 0 10.16 90) (size 1.7 1.7) (drill 1) (layers *.Cu *.Mask) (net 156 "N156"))
  (pad 10 thru_hole oval (at 2.54 10.16 90) (size 1.7 1.7) (drill 1) (layers *.Cu *.Mask) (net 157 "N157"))
  (pad 11 thru_hole oval (at 0 12.7 90) (size 1.7 1.7) (drill 1) (layers *.Cu *.Mask) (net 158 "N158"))
  (pad 12 thru_hole oval (at 2.54 12.7 90) (size 1.7 1.7) (drill 1) (layers *.Cu *.Mask) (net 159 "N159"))
  (pad 13 thru_hole oval (at 0 15.24 90) (size 1.7 1.7) (drill 1) (layers *.Cu *.Mask) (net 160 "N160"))
  (pad 14 thru_hole oval (at 2.54 15.24 90) (size 1.7 1.7) (drill 1) (layers *.Cu *.Mask) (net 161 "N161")))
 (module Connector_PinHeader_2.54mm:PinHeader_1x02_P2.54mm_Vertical (layer F.Cu) (at 85.09 94.996 90)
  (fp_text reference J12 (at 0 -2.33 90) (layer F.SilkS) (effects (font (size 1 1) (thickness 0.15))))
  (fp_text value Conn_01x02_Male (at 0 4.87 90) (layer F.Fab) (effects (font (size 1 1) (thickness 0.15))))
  (pad 1 thru_hole rect (at 0 0 90) (size 1.7 1.7) (drill 1) (layers *.Cu *.Mask) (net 15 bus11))
  (pad 2 thru_hole oval (at 0 2.54 90) (size 1.7 1.7) (drill 1) (layers *.Cu *.Mask) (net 16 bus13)))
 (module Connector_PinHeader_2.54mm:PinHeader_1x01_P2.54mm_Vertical (layer F.Cu) (at 113.792 95.25)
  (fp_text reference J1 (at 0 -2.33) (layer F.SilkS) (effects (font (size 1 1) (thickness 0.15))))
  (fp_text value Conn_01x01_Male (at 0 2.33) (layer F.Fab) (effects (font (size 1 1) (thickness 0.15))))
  (pad 1 thru_hole rect (at 0 0) (size 1.7 1.7) (drill 1) (layers *.Cu *.Mask) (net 17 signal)))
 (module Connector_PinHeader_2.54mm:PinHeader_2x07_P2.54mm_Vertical (layer F.Cu) (at 92.71 66.802 90)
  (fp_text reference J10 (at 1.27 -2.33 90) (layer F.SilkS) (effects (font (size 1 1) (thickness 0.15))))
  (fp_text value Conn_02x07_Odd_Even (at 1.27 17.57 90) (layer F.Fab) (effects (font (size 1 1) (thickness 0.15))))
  (pad 1 thru_hole rect (at 0 0 90) (size 1.7 1.7) (drill 1) (layers *.Cu *.Mask) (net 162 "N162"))
  (pad 2 thru_hole oval (at 2.54 0 90) (size 1.7 1.7) (drill 1) (layers *.Cu *.Mask) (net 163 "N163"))
  (pad 3 thru_hole oval (at 0 2.54 90) (size 1.7 1.7) (drill 1) (layers *.Cu *.Mask) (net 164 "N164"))
  (pad 4 thru_hole oval (at 2.54 2.54 90) (size 1.7 1.7) (drill 1) (layers *.Cu *.Mask) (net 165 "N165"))
  (pad 5 thru_hole oval (at 0 5.08 90) (size 1.7 1.7) (drill 1) (layers *.Cu *.Mask) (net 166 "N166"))
  (pad 6 thru_hole oval (at 2.54 5.08 90) (size 1.7 1.7) (drill 1) (layers *.Cu *.Mask) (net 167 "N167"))
  (pad 7 thru_hole oval (at 0 7.62 90) (size 1.7 1.7) (drill 1) (layers *.Cu *.Mask) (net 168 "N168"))
  (pad 8 thru_hole oval (at 2.54 7.62 90) (size 1.7 1.7) (drill 1) (layers *.Cu *.Mask) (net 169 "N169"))
  (pad 9 thru_hole oval (at 0 10.16 90) (size 1.7 1.7) (drill 1) (layers *.Cu *.Mask) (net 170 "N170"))
  (pad 10 thru_hole oval (at 2.54 10.16 90) (size 1.7 1.7) (drill 1) (layers *.Cu *.Mask) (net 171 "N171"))
  (pad 11 thru_hole oval (at 0 12.7 90) (size 1.7 1.7) (drill 1) (layers *.Cu *.Mask) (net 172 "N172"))
  (pad 12 thru_hole oval (at 2.54 12.7 90) (size 1.7 1.7) (drill 1) (layers *.Cu *.Mask) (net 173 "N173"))
  (pad 13 thru_hole oval (at 0 15.24 90) (size 1.7 1.7) (drill 1) (layers *.Cu *.Mask) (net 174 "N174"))
  (pad 14 thru_hole oval (at 2.54 15.24 90) (size 1.7 1.7) (drill 1) (layers *.Cu *.Mask) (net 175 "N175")))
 (gr_line (start 83.566 111.506) (end 83.566 57.912) (layer Edge.Cuts) (width 0.2))
 (gr_line (start 117.094 111.506) (end 83.566 111.506) (layer Edge.Cuts) (width 0.2))
 (gr_line (start 117.094 57.912) (end 117.094 111.506) (layer Edge.Cuts) (width 0.2))
 (gr_line (start 83.566 57.912) (end 117.094 57.912) (layer Edge.Cuts) (width 0.2))
 (segment (start 92.71 107.188) (end 92.71 109.728) (width 1) (layer B.Cu) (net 16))
 (segment (start 87.63 95.25) (end 87.63 102.108) (width 1) (layer B.Cu) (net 16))
 (segment (start 87.63 102.108) (end 92.71 107.188) (width 1) (layer B.Cu) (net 16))
 (segment (start 87.884 94.996) (end 87.63 95.25) (width 1) (layer B.Cu) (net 16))
 (via (at 109.22 94.996) (size 0.8) (drill 0.4) (layers F.Cu B.Cu) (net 7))
 (segment (start 105.41 106.426) (end 105.41 98.806) (width 0.25) (layer B.Cu) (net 7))
 (segment (start 105.41 98.806) (end 109.22 94.996) (width 0.25) (layer B.Cu) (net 7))
 (via (at 106.68 94.996) (size 0.8) (drill 0.4) (layers F.Cu B.Cu) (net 8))
 (segment (start 104.560001 108.116001) (end 105.41 108.966) (width 0.25) (layer B.Cu) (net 8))
 (segment (start 104.234999 107.790999) (end 104.560001 108.116001) (width 0.25) (layer B.Cu) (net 8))
 (segment (start 104.234999 98.491001) (end 104.234999 107.790999) (width 0.25) (layer B.Cu) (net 8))
 (segment (start 106.68 96.046) (end 104.234999 98.491001) (width 0.25) (layer B.Cu) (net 8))
 (segment (start 106.68 94.996) (end 106.68 96.046) (width 0.25) (layer B.Cu) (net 8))
 (via (at 104.14 94.996) (size 0.8) (drill 0.4) (layers F.Cu B.Cu) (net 9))
 (segment (start 102.87 96.266) (end 104.14 94.996) (width 0.25) (layer B.Cu) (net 9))
 (segment (start 102.87 106.426) (end 102.87 96.266) (width 0.25) (layer B.Cu) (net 9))
 (via (at 101.6 94.996) (size 0.8) (drill 0.4) (layers F.Cu B.Cu) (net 10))
 (segment (start 101.694999 95.090999) (end 101.6 94.996) (width 0.25) (layer B.Cu) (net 10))
 (segment (start 101.694999 107.790999) (end 101.694999 95.090999) (width 0.25) (layer B.Cu) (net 10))
 (segment (start 102.87 108.966) (end 101.694999 107.790999) (width 0.25) (layer B.Cu) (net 10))
 (via (at 99.06 94.996) (size 0.8) (drill 0.4) (layers F.Cu B.Cu) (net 11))
 (segment (start 100.33 96.266) (end 99.06 94.996) (width 0.25) (layer B.Cu) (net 11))
 (segment (start 100.33 106.426) (end 100.33 96.266) (width 0.25) (layer B.Cu) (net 11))
 (segment (start 99.154999 97.630999) (end 96.52 94.996) (width 0.25) (layer B.Cu) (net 12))
 (via (at 96.52 94.996) (size 0.8) (drill 0.4) (layers F.Cu B.Cu) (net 12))
 (segment (start 99.154999 107.790999) (end 99.154999 97.630999) (width 0.25) (layer B.Cu) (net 12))
 (segment (start 100.33 108.966) (end 99.154999 107.790999) (width 0.25) (layer B.Cu) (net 12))
 (via (at 93.98 94.996) (size 0.8) (drill 0.4) (layers F.Cu B.Cu) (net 13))
 (segment (start 97.79 98.806) (end 93.98 94.996) (width 0.25) (layer B.Cu) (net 13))
 (segment (start 97.79 106.426) (end 97.79 98.806) (width 0.25) (layer B.Cu) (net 13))
 (via (at 91.44 94.996) (size 0.8) (drill 0.4) (layers F.Cu B.Cu) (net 14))
 (segment (start 96.614999 100.170999) (end 91.44 94.996) (width 0.25) (layer B.Cu) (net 14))
 (segment (start 96.614999 107.790999) (end 96.614999 100.170999) (width 0.25) (layer B.Cu) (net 14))
 (segment (start 97.79 108.966) (end 96.614999 107.790999) (width 0.25) (layer B.Cu) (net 14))
 (segment (start 95.25 108.966) (end 95.25 106.671998) (width 1) (layer F.Cu) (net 15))
 (segment (start 92.964 104.902) (end 95.25 107.188) (width 1) (layer F.Cu) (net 15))
 (segment (start 89.916 104.902) (end 92.964 104.902) (width 1) (layer F.Cu) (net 15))
 (segment (start 85.344 100.33) (end 89.916 104.902) (width 1) (layer F.Cu) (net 15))
 (segment (start 85.344 95.25) (end 85.344 100.33) (width 1) (layer F.Cu) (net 15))
 (segment (start 85.09 94.996) (end 85.344 95.25) (width 1) (layer F.Cu) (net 15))
 (segment (start 108.17 102.616) (end 91.44 102.616) (width 0.25) (layer F.Cu) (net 17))
 (segment (start 109.22 102.616) (end 108.17 102.616) (width 0.25) (layer F.Cu) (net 17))
 (segment (start 91.44 101.566) (end 89.6239 99.7499) (width 0.25) (layer F.Cu) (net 17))
 (segment (start 91.44 102.616) (end 91.44 101.566) (width 0.25) (layer F.Cu) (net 17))
 (segment (start 110.27 102.616) (end 109.22 102.616) (width 0.25) (layer F.Cu) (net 17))
 (segment (start 113.792 99.094) (end 110.27 102.616) (width 0.25) (layer F.Cu) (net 17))
 (segment (start 113.792 95.25) (end 113.792 99.094) (width 0.25) (layer F.Cu) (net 17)))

